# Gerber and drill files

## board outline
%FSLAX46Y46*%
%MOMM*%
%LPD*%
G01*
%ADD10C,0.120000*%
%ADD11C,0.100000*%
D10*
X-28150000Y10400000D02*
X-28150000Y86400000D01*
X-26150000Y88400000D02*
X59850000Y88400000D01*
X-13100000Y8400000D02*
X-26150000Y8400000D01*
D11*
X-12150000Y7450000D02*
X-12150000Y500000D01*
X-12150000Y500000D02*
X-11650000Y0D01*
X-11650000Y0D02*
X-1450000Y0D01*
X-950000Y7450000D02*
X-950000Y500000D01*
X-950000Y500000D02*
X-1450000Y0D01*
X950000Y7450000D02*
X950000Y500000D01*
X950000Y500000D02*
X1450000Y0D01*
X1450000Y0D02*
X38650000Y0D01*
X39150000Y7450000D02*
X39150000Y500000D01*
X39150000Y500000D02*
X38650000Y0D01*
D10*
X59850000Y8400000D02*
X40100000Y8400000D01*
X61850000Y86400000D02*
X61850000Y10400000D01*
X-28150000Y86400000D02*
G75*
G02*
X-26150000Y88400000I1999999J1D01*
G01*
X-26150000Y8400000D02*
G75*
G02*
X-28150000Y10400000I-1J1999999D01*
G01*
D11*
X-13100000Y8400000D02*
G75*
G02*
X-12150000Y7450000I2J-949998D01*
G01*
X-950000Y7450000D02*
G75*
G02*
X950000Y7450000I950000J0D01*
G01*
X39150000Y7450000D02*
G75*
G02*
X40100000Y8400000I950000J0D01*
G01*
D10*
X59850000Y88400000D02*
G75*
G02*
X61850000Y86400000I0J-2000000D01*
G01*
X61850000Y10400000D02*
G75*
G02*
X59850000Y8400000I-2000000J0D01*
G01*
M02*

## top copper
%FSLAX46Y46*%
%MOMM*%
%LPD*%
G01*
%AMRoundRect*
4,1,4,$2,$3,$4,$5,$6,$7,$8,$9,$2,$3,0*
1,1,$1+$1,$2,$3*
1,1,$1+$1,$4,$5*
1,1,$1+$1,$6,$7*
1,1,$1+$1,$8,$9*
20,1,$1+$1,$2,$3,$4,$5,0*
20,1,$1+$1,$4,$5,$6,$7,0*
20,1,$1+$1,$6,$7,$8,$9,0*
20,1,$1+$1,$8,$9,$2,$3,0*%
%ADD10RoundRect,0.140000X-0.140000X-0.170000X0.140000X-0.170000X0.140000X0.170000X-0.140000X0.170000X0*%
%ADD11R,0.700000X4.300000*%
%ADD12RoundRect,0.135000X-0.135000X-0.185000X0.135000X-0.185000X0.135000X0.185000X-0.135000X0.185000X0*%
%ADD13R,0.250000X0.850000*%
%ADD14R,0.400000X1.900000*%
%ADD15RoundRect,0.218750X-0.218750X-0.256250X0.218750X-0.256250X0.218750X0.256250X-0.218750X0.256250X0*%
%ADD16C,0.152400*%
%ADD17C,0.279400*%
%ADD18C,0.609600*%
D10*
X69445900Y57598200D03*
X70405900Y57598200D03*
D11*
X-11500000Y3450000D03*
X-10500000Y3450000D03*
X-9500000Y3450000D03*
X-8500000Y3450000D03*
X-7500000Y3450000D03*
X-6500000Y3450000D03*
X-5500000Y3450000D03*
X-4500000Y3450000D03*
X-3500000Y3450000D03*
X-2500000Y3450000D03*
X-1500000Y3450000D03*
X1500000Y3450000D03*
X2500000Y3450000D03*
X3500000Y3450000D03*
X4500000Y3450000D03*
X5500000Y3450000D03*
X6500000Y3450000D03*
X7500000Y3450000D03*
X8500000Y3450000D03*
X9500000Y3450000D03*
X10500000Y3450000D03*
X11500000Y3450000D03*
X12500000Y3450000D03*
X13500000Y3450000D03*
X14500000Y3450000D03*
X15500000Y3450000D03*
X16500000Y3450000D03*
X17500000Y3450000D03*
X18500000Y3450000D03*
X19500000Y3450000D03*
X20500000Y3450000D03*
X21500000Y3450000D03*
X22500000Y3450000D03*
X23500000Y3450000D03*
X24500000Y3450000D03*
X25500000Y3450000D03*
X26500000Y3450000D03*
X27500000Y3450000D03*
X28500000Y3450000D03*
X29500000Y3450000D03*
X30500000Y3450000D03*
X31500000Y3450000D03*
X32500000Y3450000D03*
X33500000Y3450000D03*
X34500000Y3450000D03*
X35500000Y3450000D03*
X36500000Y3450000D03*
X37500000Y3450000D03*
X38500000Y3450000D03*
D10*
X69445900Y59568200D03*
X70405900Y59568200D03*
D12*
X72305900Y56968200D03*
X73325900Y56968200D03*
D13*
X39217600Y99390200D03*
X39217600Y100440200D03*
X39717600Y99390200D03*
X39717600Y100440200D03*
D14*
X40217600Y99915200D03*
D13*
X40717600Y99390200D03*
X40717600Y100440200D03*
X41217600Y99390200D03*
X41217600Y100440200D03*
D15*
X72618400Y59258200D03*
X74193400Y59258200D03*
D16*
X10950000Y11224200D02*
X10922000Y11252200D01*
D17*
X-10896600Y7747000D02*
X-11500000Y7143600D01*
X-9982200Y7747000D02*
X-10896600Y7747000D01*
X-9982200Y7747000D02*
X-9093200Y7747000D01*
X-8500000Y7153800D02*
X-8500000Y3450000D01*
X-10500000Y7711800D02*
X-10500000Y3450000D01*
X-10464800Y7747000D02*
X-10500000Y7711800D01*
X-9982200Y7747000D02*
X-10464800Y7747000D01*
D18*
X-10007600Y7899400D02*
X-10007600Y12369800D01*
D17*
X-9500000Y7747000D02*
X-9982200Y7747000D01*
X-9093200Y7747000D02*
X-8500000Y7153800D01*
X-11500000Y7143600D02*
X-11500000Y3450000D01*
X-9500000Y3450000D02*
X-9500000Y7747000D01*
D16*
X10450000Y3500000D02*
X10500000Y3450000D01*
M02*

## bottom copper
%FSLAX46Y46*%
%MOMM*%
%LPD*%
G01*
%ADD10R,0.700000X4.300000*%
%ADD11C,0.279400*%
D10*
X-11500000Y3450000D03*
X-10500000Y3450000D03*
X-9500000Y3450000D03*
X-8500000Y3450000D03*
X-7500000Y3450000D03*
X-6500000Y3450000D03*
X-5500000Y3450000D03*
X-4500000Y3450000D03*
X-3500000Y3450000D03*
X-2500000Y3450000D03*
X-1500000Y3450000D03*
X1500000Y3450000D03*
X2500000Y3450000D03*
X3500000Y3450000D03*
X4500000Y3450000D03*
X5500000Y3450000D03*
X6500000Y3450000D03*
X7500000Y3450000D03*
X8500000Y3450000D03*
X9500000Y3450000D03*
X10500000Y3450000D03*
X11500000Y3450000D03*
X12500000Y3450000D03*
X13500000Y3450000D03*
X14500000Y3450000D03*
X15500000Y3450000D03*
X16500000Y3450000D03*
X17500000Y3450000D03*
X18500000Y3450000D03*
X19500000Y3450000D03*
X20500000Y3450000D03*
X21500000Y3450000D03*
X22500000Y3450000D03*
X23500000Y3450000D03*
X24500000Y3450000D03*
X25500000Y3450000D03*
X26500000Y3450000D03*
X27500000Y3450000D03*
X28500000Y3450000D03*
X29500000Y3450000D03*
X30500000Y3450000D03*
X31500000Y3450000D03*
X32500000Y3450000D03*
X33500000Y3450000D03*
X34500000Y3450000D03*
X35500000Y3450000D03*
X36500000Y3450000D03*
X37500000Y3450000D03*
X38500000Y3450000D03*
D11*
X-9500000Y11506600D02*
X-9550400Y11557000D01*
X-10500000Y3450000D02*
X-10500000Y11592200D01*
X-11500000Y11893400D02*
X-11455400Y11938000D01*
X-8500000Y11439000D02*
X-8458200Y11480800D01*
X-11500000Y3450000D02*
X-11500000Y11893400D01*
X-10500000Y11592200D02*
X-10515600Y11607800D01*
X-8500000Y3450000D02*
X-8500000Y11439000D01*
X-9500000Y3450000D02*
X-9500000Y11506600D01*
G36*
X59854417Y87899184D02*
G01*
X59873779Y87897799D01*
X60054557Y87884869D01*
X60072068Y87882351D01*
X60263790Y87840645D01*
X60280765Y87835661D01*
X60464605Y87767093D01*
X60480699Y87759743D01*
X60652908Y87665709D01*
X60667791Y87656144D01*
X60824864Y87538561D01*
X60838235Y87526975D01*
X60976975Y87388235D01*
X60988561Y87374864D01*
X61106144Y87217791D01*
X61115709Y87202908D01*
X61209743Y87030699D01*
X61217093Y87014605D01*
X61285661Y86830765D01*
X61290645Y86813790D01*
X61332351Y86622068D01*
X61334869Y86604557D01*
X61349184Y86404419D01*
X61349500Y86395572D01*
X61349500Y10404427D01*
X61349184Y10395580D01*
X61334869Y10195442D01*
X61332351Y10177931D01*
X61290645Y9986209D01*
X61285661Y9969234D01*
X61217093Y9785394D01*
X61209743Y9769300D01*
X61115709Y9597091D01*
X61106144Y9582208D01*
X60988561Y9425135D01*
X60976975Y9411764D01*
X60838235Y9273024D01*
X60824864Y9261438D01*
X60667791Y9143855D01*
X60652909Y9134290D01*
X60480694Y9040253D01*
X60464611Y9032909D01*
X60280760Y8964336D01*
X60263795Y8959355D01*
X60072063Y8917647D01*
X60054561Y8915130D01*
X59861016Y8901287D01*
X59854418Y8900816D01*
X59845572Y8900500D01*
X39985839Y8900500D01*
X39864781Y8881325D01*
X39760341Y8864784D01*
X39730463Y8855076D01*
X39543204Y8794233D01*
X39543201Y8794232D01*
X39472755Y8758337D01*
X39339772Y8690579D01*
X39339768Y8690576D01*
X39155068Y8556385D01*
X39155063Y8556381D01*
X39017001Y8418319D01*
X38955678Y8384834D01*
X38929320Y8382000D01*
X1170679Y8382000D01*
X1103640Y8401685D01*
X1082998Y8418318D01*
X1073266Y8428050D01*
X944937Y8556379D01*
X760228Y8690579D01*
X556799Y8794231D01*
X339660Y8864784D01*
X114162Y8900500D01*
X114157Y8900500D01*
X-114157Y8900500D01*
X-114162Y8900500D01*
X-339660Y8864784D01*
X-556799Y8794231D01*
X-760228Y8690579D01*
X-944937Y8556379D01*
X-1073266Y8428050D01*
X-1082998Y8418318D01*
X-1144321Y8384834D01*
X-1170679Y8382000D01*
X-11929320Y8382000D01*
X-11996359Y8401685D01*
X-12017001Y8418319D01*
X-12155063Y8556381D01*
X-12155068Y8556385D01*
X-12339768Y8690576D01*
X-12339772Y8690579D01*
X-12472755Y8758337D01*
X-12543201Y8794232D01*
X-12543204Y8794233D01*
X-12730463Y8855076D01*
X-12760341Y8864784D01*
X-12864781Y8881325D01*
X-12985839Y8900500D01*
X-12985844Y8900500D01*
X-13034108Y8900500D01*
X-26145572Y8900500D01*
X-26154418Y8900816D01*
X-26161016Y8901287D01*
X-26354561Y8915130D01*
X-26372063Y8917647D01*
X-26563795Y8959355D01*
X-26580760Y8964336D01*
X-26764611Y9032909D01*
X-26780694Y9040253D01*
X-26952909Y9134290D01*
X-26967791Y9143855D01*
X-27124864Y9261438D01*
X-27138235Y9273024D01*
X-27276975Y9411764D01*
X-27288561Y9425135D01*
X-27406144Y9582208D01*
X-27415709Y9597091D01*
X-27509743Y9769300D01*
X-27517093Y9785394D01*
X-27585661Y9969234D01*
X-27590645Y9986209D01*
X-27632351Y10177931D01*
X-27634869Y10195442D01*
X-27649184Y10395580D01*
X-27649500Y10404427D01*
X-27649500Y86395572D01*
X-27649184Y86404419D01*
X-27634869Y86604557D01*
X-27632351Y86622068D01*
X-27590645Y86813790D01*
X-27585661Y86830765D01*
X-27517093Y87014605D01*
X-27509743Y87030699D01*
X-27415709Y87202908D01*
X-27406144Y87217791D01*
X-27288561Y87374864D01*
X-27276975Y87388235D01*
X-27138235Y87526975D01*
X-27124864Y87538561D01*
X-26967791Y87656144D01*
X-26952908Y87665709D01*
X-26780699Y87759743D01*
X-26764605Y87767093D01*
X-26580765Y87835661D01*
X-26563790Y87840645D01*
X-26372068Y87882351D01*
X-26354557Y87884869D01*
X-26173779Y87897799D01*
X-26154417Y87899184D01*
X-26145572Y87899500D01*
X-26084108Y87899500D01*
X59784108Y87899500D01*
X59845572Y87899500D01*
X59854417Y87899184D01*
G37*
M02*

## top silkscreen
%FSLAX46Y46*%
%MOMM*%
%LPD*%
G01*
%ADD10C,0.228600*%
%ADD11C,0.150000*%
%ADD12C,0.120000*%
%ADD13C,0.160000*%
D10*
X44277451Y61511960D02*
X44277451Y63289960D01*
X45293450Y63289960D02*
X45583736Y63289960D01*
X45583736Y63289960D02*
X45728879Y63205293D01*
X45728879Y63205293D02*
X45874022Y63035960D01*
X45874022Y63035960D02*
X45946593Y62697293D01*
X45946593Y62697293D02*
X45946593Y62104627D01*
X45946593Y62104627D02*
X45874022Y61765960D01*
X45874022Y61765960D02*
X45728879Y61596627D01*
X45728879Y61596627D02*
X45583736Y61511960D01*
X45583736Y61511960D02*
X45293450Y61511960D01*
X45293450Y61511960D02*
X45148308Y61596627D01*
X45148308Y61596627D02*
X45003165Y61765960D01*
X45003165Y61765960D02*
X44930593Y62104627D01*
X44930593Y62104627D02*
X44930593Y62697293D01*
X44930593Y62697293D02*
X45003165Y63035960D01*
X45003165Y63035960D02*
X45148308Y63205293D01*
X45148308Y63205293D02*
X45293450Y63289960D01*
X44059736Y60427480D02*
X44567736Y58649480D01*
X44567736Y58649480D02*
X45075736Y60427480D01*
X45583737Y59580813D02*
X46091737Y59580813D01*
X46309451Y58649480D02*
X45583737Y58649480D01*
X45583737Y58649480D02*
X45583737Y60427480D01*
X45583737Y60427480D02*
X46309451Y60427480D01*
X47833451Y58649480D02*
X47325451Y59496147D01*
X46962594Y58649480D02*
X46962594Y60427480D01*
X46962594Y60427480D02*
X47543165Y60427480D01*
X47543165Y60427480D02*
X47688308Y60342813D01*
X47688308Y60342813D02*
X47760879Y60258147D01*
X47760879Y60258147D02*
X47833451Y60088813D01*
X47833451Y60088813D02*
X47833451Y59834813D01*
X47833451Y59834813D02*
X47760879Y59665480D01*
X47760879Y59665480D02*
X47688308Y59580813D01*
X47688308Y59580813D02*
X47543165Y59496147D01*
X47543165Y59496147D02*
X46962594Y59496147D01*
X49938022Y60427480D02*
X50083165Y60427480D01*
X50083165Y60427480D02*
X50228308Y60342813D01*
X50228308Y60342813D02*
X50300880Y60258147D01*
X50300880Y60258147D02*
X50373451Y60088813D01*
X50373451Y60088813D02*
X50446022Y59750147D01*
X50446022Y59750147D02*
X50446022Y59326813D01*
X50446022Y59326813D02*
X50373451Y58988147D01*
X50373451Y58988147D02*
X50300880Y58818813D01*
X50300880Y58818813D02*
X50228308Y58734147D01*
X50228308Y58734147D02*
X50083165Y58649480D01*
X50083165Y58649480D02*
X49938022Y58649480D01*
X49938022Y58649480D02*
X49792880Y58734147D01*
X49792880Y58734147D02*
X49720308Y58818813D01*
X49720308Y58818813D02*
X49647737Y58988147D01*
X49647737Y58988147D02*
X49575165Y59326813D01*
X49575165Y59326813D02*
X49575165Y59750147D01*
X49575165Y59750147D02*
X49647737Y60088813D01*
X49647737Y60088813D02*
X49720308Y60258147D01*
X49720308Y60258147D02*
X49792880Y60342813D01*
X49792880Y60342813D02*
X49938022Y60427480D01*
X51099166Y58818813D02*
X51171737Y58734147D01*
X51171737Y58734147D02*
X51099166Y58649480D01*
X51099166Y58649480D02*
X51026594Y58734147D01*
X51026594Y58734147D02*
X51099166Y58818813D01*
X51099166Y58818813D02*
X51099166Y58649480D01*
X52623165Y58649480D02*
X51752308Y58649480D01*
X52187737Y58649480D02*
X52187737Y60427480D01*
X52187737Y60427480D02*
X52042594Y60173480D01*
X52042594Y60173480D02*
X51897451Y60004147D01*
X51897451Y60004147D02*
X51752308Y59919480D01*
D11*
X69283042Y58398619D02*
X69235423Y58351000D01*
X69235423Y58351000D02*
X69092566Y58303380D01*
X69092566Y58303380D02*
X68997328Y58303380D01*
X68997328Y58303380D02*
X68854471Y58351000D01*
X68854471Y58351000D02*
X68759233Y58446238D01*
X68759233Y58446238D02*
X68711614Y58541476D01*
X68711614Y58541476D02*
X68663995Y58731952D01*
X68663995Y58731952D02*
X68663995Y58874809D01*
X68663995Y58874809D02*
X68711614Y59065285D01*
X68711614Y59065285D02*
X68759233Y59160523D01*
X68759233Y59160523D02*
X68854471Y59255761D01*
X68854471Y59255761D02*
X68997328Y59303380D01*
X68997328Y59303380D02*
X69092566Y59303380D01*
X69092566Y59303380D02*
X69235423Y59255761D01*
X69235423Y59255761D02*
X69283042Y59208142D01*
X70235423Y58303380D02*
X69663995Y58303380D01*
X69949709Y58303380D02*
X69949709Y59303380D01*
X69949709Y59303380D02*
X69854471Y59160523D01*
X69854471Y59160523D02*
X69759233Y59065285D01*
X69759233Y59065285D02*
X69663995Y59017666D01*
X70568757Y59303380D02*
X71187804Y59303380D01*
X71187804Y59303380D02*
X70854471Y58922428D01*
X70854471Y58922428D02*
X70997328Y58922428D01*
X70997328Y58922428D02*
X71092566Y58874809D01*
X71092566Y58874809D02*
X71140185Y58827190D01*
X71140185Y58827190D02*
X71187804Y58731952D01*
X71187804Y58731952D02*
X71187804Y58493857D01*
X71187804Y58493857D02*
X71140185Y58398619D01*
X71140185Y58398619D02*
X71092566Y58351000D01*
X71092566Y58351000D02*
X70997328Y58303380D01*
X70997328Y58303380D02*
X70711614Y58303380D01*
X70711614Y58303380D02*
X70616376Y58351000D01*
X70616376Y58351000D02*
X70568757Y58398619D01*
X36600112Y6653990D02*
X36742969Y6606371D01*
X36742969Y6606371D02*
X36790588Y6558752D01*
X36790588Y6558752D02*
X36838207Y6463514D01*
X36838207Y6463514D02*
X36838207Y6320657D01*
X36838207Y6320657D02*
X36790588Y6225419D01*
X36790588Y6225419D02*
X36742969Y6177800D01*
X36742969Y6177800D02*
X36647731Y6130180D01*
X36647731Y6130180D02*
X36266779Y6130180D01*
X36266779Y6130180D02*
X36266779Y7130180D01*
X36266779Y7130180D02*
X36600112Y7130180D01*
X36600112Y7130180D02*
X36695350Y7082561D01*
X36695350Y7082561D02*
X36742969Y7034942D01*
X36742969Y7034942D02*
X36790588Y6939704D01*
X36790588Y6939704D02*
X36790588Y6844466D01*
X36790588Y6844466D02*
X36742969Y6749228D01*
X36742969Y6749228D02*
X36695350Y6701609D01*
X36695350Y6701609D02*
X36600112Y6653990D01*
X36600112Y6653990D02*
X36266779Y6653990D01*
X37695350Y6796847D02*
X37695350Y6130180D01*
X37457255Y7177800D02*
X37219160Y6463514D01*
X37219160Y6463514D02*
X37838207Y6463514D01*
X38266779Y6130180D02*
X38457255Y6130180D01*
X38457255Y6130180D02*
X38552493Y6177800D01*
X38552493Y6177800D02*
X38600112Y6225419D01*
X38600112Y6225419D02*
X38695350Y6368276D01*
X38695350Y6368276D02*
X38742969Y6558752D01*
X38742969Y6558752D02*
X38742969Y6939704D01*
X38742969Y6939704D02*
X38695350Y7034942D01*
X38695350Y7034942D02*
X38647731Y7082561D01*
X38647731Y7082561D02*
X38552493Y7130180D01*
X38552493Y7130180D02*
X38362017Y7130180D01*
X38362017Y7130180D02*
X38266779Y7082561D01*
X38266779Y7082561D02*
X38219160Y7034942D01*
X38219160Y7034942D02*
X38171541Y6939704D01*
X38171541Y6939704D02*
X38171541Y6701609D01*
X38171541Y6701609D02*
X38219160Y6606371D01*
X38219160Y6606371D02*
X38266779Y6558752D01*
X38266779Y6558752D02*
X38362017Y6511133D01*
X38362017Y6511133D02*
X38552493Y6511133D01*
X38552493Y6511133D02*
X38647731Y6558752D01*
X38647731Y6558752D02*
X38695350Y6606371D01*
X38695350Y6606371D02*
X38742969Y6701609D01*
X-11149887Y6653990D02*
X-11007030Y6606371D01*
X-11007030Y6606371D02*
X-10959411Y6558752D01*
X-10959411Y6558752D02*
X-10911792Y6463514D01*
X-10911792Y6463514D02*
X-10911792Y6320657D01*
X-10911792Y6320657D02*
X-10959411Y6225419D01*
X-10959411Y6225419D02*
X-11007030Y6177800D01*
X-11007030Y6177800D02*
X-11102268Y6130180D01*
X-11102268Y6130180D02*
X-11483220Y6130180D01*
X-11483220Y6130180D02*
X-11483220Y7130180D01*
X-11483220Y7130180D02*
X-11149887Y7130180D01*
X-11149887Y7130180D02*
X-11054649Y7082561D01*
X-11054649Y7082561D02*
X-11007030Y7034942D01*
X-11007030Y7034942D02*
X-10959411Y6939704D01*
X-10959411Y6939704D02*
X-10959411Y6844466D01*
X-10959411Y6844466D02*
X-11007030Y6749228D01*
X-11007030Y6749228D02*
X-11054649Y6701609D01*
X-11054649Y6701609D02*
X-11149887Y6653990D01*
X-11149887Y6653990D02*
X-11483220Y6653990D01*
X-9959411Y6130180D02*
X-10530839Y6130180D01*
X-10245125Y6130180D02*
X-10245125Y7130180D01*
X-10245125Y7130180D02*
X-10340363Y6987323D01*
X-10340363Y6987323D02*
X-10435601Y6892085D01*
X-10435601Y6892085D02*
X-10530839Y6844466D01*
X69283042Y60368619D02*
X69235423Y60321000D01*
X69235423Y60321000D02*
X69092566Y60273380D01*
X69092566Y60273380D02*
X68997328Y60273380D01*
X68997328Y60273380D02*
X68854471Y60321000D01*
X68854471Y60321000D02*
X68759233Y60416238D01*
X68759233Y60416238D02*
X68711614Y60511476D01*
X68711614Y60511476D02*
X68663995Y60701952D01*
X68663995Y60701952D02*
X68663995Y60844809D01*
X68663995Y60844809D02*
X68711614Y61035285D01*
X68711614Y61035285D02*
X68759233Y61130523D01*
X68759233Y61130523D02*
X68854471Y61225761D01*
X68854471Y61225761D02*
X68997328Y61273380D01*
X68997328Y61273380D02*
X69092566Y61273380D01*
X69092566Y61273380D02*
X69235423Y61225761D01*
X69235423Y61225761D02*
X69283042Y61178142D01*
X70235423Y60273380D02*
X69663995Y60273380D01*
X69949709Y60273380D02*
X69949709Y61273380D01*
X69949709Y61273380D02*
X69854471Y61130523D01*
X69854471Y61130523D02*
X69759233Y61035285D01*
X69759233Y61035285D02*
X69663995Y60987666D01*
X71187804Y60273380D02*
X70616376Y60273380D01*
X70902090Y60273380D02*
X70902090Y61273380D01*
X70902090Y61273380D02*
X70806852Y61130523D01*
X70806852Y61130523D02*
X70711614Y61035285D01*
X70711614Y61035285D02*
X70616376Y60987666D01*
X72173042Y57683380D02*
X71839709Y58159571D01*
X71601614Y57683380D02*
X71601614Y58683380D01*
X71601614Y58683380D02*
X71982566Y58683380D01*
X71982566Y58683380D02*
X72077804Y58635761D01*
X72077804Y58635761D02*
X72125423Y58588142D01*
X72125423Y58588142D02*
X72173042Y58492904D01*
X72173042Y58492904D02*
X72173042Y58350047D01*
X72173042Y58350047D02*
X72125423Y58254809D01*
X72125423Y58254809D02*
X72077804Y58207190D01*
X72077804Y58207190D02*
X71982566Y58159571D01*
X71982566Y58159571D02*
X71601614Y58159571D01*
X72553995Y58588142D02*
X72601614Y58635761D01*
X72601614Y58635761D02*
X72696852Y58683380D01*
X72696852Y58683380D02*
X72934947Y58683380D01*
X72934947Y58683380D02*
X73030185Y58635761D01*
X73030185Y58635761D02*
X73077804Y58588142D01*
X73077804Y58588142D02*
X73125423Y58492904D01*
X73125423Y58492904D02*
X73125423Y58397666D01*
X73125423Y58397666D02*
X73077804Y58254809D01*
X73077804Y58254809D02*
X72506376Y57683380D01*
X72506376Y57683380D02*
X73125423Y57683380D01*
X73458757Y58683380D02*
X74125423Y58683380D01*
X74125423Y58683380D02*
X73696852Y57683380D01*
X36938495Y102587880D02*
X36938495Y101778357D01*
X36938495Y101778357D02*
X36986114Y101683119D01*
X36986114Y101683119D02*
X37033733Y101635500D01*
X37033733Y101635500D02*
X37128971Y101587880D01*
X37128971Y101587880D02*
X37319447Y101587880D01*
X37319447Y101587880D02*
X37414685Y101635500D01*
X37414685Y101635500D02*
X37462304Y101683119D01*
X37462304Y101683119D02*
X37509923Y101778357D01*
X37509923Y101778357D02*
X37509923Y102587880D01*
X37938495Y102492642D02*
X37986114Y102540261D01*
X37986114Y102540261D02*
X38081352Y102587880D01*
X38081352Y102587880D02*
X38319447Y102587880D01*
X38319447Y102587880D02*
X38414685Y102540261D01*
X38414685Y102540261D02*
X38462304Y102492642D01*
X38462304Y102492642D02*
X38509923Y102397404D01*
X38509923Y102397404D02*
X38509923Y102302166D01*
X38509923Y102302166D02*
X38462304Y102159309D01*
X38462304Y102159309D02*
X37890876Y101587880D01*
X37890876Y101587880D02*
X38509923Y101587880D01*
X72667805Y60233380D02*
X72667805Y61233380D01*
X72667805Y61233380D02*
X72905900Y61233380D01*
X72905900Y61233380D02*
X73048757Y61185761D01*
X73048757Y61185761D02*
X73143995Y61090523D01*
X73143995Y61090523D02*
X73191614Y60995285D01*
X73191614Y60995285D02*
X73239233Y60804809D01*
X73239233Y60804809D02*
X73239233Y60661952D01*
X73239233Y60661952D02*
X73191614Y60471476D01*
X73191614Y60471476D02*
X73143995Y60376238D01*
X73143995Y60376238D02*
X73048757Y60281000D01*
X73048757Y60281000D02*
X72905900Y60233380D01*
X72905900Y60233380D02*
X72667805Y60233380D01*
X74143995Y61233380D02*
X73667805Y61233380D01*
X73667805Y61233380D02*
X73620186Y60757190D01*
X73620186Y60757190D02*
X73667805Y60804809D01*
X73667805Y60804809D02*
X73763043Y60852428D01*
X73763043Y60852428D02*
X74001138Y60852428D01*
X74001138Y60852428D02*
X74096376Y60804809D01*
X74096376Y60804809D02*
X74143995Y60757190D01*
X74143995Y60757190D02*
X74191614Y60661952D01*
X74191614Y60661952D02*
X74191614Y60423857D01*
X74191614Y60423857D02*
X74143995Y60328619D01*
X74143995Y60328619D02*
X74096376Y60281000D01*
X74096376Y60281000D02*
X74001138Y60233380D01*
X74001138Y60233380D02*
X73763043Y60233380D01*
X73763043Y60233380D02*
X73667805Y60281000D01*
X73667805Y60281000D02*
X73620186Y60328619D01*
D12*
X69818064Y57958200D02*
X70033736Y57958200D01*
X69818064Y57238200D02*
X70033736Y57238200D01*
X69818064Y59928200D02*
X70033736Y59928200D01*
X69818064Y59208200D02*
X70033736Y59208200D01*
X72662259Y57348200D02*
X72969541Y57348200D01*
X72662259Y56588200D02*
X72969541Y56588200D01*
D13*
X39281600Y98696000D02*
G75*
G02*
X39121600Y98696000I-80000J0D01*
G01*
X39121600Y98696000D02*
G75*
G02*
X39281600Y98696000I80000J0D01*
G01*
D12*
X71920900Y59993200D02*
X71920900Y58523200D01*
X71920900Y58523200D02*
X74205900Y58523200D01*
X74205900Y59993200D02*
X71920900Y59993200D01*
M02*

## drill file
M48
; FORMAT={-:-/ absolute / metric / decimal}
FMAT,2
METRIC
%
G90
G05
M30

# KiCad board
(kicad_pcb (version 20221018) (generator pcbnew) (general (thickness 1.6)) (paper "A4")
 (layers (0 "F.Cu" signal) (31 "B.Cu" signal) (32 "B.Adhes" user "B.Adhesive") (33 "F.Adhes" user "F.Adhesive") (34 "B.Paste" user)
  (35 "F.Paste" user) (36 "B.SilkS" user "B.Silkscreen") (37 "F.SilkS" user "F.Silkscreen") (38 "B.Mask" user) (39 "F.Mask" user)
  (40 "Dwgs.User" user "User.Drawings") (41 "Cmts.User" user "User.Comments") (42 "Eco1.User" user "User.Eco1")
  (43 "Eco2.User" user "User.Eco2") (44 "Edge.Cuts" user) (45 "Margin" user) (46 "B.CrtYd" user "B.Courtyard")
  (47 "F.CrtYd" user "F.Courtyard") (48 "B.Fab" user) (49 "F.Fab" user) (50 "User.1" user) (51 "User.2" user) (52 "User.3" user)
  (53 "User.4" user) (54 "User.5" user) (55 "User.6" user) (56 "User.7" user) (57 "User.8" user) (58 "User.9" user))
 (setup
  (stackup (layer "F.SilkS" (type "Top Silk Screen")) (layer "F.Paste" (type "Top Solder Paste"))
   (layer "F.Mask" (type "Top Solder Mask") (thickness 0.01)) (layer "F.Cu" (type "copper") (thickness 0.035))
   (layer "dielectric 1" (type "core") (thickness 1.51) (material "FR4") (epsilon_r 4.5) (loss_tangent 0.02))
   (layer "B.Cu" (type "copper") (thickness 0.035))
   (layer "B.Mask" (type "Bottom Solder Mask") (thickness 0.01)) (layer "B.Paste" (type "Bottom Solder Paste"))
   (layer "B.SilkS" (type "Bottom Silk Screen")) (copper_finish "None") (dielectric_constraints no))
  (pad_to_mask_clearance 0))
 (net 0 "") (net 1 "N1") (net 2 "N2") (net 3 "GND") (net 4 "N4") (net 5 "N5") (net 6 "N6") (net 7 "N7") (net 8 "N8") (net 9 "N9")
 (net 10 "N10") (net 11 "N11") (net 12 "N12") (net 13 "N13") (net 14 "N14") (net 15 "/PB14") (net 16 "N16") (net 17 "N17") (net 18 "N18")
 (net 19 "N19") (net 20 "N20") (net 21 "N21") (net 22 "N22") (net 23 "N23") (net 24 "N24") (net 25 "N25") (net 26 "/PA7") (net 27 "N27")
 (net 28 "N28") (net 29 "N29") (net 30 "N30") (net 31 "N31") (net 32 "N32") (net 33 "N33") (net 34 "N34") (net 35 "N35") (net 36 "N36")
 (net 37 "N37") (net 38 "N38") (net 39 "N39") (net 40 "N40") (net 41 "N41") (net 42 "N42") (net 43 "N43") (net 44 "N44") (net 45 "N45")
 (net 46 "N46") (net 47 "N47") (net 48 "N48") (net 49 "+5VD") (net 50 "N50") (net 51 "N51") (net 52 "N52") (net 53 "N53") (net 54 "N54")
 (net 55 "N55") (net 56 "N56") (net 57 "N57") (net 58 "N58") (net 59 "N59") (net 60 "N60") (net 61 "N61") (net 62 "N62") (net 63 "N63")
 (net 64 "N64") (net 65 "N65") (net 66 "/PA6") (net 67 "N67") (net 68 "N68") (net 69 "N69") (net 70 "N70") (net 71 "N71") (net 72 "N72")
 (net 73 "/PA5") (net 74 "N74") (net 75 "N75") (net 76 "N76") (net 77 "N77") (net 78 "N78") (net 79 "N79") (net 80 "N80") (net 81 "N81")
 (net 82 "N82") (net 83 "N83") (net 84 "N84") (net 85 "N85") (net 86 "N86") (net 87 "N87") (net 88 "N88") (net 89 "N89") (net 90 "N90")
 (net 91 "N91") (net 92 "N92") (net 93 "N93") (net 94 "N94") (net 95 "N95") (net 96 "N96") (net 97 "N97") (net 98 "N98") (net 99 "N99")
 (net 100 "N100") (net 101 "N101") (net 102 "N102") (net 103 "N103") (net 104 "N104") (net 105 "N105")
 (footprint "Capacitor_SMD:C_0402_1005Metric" (layer "F.Cu") (at 69.9259 -57.5982)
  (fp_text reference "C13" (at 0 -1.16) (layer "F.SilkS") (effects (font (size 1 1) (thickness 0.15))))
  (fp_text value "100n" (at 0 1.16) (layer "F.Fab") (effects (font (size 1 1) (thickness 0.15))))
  (fp_line (start -0.107836 -0.36) (end 0.107836 -0.36) (stroke (width 0.12) (type solid)) (layer "F.SilkS"))
  (fp_line (start -0.107836 0.36) (end 0.107836 0.36) (stroke (width 0.12) (type solid)) (layer "F.SilkS"))
  (pad "1" smd roundrect (at -0.48 0) (size 0.56 0.62) (layers "F.Cu" "F.Paste" "F.Mask") (roundrect_rratio 0.25) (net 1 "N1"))
  (pad "2" smd roundrect (at 0.48 0) (size 0.56 0.62) (layers "F.Cu" "F.Paste" "F.Mask") (roundrect_rratio 0.25) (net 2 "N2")))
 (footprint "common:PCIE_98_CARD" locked (layer "F.Cu") (at 0 0)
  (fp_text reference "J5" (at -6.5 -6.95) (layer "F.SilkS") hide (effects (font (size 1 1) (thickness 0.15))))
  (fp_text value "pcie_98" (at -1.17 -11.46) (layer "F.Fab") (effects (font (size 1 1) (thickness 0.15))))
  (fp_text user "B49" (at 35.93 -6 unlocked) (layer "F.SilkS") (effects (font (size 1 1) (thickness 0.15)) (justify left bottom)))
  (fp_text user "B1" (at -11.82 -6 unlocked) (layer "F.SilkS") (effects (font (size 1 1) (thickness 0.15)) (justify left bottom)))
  (fp_line (start -28.15 -10.4) (end -28.15 -86.4) (stroke (width 0.12) (type default)) (layer "Edge.Cuts"))
  (fp_line (start -26.15 -88.4) (end 59.85 -88.4) (stroke (width 0.12) (type default)) (layer "Edge.Cuts"))
  (fp_line (start -13.1 -8.4) (end -26.15 -8.4) (stroke (width 0.12) (type default)) (layer "Edge.Cuts"))
  (fp_line (start -12.15 -7.45) (end -12.15 -0.5) (stroke (width 0.1) (type solid)) (layer "Edge.Cuts"))
  (fp_line (start -12.15 -0.5) (end -11.65 0) (stroke (width 0.1) (type solid)) (layer "Edge.Cuts"))
  (fp_line (start -11.65 0) (end -1.45 0) (stroke (width 0.1) (type solid)) (layer "Edge.Cuts"))
  (fp_line (start -0.95 -7.45) (end -0.95 -0.5) (stroke (width 0.1) (type solid)) (layer "Edge.Cuts"))
  (fp_line (start -0.95 -0.5) (end -1.45 0) (stroke (width 0.1) (type solid)) (layer "Edge.Cuts"))
  (fp_line (start 0.95 -7.45) (end 0.95 -0.5) (stroke (width 0.1) (type solid)) (layer "Edge.Cuts"))
  (fp_line (start 0.95 -0.5) (end 1.45 0) (stroke (width 0.1) (type solid)) (layer "Edge.Cuts"))
  (fp_line (start 1.45 0) (end 38.65 0) (stroke (width 0.1) (type solid)) (layer "Edge.Cuts"))
  (fp_line (start 39.15 -7.45) (end 39.15 -0.5) (stroke (width 0.1) (type solid)) (layer "Edge.Cuts"))
  (fp_line (start 39.15 -0.5) (end 38.65 0) (stroke (width 0.1) (type solid)) (layer "Edge.Cuts"))
  (fp_line (start 59.85 -8.4) (end 40.1 -8.4) (stroke (width 0.12) (type default)) (layer "Edge.Cuts"))
  (fp_line (start 61.85 -86.4) (end 61.85 -10.4) (stroke (width 0.12) (type default)) (layer "Edge.Cuts"))
  (fp_arc (start -28.15 -86.4) (mid -27.564214 -87.814214) (end -26.15 -88.4) (stroke (width 0.12) (type default)) (layer "Edge.Cuts"))
  (fp_arc (start -26.15 -8.4) (mid -27.564214 -8.985786) (end -28.15 -10.4) (stroke (width 0.12) (type default)) (layer "Edge.Cuts"))
  (fp_arc (start -13.1 -8.4) (mid -12.428248 -8.121752) (end -12.15 -7.45) (stroke (width 0.1) (type default)) (layer "Edge.Cuts"))
  (fp_arc (start -0.95 -7.45) (mid 0 -8.4) (end 0.95 -7.45) (stroke (width 0.1) (type solid)) (layer "Edge.Cuts"))
  (fp_arc (start 39.15 -7.45) (mid 39.428248 -8.121752) (end 40.1 -8.4) (stroke (width 0.1) (type default)) (layer "Edge.Cuts"))
  (fp_arc (start 59.85 -88.4) (mid 61.264214 -87.814214) (end 61.85 -86.4) (stroke (width 0.12) (type default)) (layer "Edge.Cuts"))
  (fp_arc (start 61.85 -10.4) (mid 61.264214 -8.985786) (end 59.85 -8.4) (stroke (width 0.12) (type default)) (layer "Edge.Cuts"))
  (pad "A1" connect rect locked (at -11.5 -3.45) (size 0.7 4.3) (layers "B.Cu" "B.Mask") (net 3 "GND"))
  (pad "A2" connect rect locked (at -10.5 -3.45) (size 0.7 4.3) (layers "B.Cu" "B.Mask") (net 3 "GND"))
  (pad "A3" connect rect locked (at -9.5 -3.45) (size 0.7 4.3) (layers "B.Cu" "B.Mask") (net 3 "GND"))
  (pad "A4" connect rect locked (at -8.5 -3.45) (size 0.7 4.3) (layers "B.Cu" "B.Mask") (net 3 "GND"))
  (pad "A5" connect rect locked (at -7.5 -3.45) (size 0.7 4.3) (layers "B.Cu" "B.Mask") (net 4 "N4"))
  (pad "A6" connect rect locked (at -6.5 -3.45) (size 0.7 4.3) (layers "B.Cu" "B.Mask") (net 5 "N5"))
  (pad "A7" connect rect locked (at -5.5 -3.45) (size 0.7 4.3) (layers "B.Cu" "B.Mask") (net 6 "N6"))
  (pad "A8" connect rect locked (at -4.5 -3.45) (size 0.7 4.3) (layers "B.Cu" "B.Mask") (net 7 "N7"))
  (pad "A9" connect rect locked (at -3.5 -3.45) (size 0.7 4.3) (layers "B.Cu" "B.Mask") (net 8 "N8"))
  (pad "A10" connect rect locked (at -2.5 -3.45) (size 0.7 4.3) (layers "B.Cu" "B.Mask") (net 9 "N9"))
  (pad "A11" connect rect locked (at -1.5 -3.45) (size 0.7 4.3) (layers "B.Cu" "B.Mask") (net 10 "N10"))
  (pad "A12" connect rect locked (at 1.5 -3.45) (size 0.7 4.3) (layers "B.Cu" "B.Mask") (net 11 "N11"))
  (pad "A13" connect rect locked (at 2.5 -3.45) (size 0.7 4.3) (layers "B.Cu" "B.Mask") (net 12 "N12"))
  (pad "A14" connect rect locked (at 3.5 -3.45) (size 0.7 4.3) (layers "B.Cu" "B.Mask") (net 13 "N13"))
  (pad "A15" connect rect locked (at 4.5 -3.45) (size 0.7 4.3) (layers "B.Cu" "B.Mask") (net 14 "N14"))
  (pad "A16" connect rect locked (at 5.5 -3.45) (size 0.7 4.3) (layers "B.Cu" "B.Mask") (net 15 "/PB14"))
  (pad "A17" connect rect locked (at 6.5 -3.45) (size 0.7 4.3) (layers "B.Cu" "B.Mask") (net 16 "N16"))
  (pad "A18" connect rect locked (at 7.5 -3.45) (size 0.7 4.3) (layers "B.Cu" "B.Mask") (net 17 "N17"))
  (pad "A19" connect rect locked (at 8.5 -3.45) (size 0.7 4.3) (layers "B.Cu" "B.Mask") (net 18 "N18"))
  (pad "A20" connect rect locked (at 9.5 -3.45) (size 0.7 4.3) (layers "B.Cu" "B.Mask") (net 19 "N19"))
  (pad "A21" connect rect locked (at 10.5 -3.45) (size 0.7 4.3) (layers "B.Cu" "B.Mask") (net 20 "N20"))
  (pad "A22" connect rect locked (at 11.5 -3.45) (size 0.7 4.3) (layers "B.Cu" "B.Mask") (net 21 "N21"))
  (pad "A23" connect rect locked (at 12.5 -3.45) (size 0.7 4.3) (layers "B.Cu" "B.Mask") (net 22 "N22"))
  (pad "A24" connect rect locked (at 13.5 -3.45) (size 0.7 4.3) (layers "B.Cu" "B.Mask") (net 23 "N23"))
  (pad "A25" connect rect locked (at 14.5 -3.45) (size 0.7 4.3) (layers "B.Cu" "B.Mask") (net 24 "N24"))
  (pad "A26" connect rect locked (at 15.5 -3.45) (size 0.7 4.3) (layers "B.Cu" "B.Mask") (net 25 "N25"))
  (pad "A27" connect rect locked (at 16.5 -3.45) (size 0.7 4.3) (layers "B.Cu" "B.Mask") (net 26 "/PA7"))
  (pad "A28" connect rect locked (at 17.5 -3.45) (size 0.7 4.3) (layers "B.Cu" "B.Mask") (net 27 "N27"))
  (pad "A29" connect rect locked (at 18.5 -3.45) (size 0.7 4.3) (layers "B.Cu" "B.Mask") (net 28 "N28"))
  (pad "A30" connect rect locked (at 19.5 -3.45) (size 0.7 4.3) (layers "B.Cu" "B.Mask") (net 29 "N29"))
  (pad "A31" connect rect locked (at 20.5 -3.45) (size 0.7 4.3) (layers "B.Cu" "B.Mask") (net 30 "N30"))
  (pad "A32" connect rect locked (at 21.5 -3.45) (size 0.7 4.3) (layers "B.Cu" "B.Mask") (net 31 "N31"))
  (pad "A33" connect rect locked (at 22.5 -3.45) (size 0.7 4.3) (layers "B.Cu" "B.Mask") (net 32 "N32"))
  (pad "A34" connect rect locked (at 23.5 -3.45) (size 0.7 4.3) (layers "B.Cu" "B.Mask") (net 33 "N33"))
  (pad "A35" connect rect locked (at 24.5 -3.45) (size 0.7 4.3) (layers "B.Cu" "B.Mask") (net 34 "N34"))
  (pad "A36" connect rect locked (at 25.5 -3.45) (size 0.7 4.3) (layers "B.Cu" "B.Mask") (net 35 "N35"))
  (pad "A37" connect rect locked (at 26.5 -3.45) (size 0.7 4.3) (layers "B.Cu" "B.Mask") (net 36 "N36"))
  (pad "A38" connect rect locked (at 27.5 -3.45) (size 0.7 4.3) (layers "B.Cu" "B.Mask") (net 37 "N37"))
  (pad "A39" connect rect locked (at 28.5 -3.45) (size 0.7 4.3) (layers "B.Cu" "B.Mask") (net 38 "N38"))
  (pad "A40" connect rect locked (at 29.5 -3.45) (size 0.7 4.3) (layers "B.Cu" "B.Mask") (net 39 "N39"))
  (pad "A41" connect rect locked (at 30.5 -3.45) (size 0.7 4.3) (layers "B.Cu" "B.Mask") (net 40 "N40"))
  (pad "A42" connect rect locked (at 31.5 -3.45) (size 0.7 4.3) (layers "B.Cu" "B.Mask") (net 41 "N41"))
  (pad "A43" connect rect locked (at 32.5 -3.45) (size 0.7 4.3) (layers "B.Cu" "B.Mask") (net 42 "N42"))
  (pad "A44" connect rect locked (at 33.5 -3.45) (size 0.7 4.3) (layers "B.Cu" "B.Mask") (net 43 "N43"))
  (pad "A45" connect rect locked (at 34.5 -3.45) (size 0.7 4.3) (layers "B.Cu" "B.Mask") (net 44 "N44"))
  (pad "A46" connect rect locked (at 35.5 -3.45) (size 0.7 4.3) (layers "B.Cu" "B.Mask") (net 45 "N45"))
  (pad "A47" connect rect locked (at 36.5 -3.45) (size 0.7 4.3) (layers "B.Cu" "B.Mask") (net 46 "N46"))
  (pad "A48" connect rect locked (at 37.5 -3.45) (size 0.7 4.3) (layers "B.Cu" "B.Mask") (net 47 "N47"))
  (pad "A49" connect rect locked (at 38.5 -3.45) (size 0.7 4.3) (layers "B.Cu" "B.Mask") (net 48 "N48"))
  (pad "B1" connect rect locked (at -11.5 -3.45) (size 0.7 4.3) (layers "F.Cu" "F.Mask") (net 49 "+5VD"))
  (pad "B2" connect rect locked (at -10.5 -3.45) (size 0.7 4.3) (layers "F.Cu" "F.Mask") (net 49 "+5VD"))
  (pad "B3" connect rect locked (at -9.5 -3.45) (size 0.7 4.3) (layers "F.Cu" "F.Mask") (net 49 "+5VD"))
  (pad "B4" connect rect locked (at -8.5 -3.45) (size 0.7 4.3) (layers "F.Cu" "F.Mask") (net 49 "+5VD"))
  (pad "B5" connect rect locked (at -7.5 -3.45) (size 0.7 4.3) (layers "F.Cu" "F.Mask") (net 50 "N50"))
  (pad "B6" connect rect locked (at -6.5 -3.45) (size 0.7 4.3) (layers "F.Cu" "F.Mask") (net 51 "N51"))
  (pad "B7" connect rect locked (at -5.5 -3.45) (size 0.7 4.3) (layers "F.Cu" "F.Mask") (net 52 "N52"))
  (pad "B8" connect rect locked (at -4.5 -3.45) (size 0.7 4.3) (layers "F.Cu" "F.Mask") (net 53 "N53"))
  (pad "B9" connect rect locked (at -3.5 -3.45) (size 0.7 4.3) (layers "F.Cu" "F.Mask") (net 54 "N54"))
  (pad "B10" connect rect locked (at -2.5 -3.45) (size 0.7 4.3) (layers "F.Cu" "F.Mask") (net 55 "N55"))
  (pad "B11" connect rect locked (at -1.5 -3.45) (size 0.7 4.3) (layers "F.Cu" "F.Mask") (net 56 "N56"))
  (pad "B12" connect rect locked (at 1.5 -3.45) (size 0.7 4.3) (layers "F.Cu" "F.Mask") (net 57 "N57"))
  (pad "B13" connect rect locked (at 2.5 -3.45) (size 0.7 4.3) (layers "F.Cu" "F.Mask") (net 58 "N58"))
  (pad "B14" connect rect locked (at 3.5 -3.45) (size 0.7 4.3) (layers "F.Cu" "F.Mask") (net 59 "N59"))
  (pad "B15" connect rect locked (at 4.5 -3.45) (size 0.7 4.3) (layers "F.Cu" "F.Mask") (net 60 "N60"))
  (pad "B16" connect rect locked (at 5.5 -3.45) (size 0.7 4.3) (layers "F.Cu" "F.Mask") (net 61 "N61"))
  (pad "B17" connect rect locked (at 6.5 -3.45) (size 0.7 4.3) (layers "F.Cu" "F.Mask") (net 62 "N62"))
  (pad "B18" connect rect locked (at 7.5 -3.45) (size 0.7 4.3) (layers "F.Cu" "F.Mask") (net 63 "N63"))
  (pad "B19" connect rect locked (at 8.5 -3.45) (size 0.7 4.3) (layers "F.Cu" "F.Mask") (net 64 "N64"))
  (pad "B20" connect rect locked (at 9.5 -3.45) (size 0.7 4.3) (layers "F.Cu" "F.Mask") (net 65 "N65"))
  (pad "B21" connect rect locked (at 10.5 -3.45) (size 0.7 4.3) (layers "F.Cu" "F.Mask") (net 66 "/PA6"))
  (pad "B22" connect rect locked (at 11.5 -3.45) (size 0.7 4.3) (layers "F.Cu" "F.Mask") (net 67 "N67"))
  (pad "B23" connect rect locked (at 12.5 -3.45) (size 0.7 4.3) (layers "F.Cu" "F.Mask") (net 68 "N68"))
  (pad "B24" connect rect locked (at 13.5 -3.45) (size 0.7 4.3) (layers "F.Cu" "F.Mask") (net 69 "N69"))
  (pad "B25" connect rect locked (at 14.5 -3.45) (size 0.7 4.3) (layers "F.Cu" "F.Mask") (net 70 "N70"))
  (pad "B26" connect rect locked (at 15.5 -3.45) (size 0.7 4.3) (layers "F.Cu" "F.Mask") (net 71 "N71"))
  (pad "B27" connect rect locked (at 16.5 -3.45) (size 0.7 4.3) (layers "F.Cu" "F.Mask") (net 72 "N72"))
  (pad "B28" connect rect locked (at 17.5 -3.45) (size 0.7 4.3) (layers "F.Cu" "F.Mask") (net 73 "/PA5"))
  (pad "B29" connect rect locked (at 18.5 -3.45) (size 0.7 4.3) (layers "F.Cu" "F.Mask") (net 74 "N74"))
  (pad "B30" connect rect locked (at 19.5 -3.45) (size 0.7 4.3) (layers "F.Cu" "F.Mask") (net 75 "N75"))
  (pad "B31" connect rect locked (at 20.5 -3.45) (size 0.7 4.3) (layers "F.Cu" "F.Mask") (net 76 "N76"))
  (pad "B32" connect rect locked (at 21.5 -3.45) (size 0.7 4.3) (layers "F.Cu" "F.Mask") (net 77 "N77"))
  (pad "B33" connect rect locked (at 22.5 -3.45) (size 0.7 4.3) (layers "F.Cu" "F.Mask") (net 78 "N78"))
  (pad "B34" connect rect locked (at 23.5 -3.45) (size 0.7 4.3) (layers "F.Cu" "F.Mask") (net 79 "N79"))
  (pad "B35" connect rect locked (at 24.5 -3.45) (size 0.7 4.3) (layers "F.Cu" "F.Mask") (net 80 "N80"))
  (pad "B36" connect rect locked (at 25.5 -3.45) (size 0.7 4.3) (layers "F.Cu" "F.Mask") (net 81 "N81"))
  (pad "B37" connect rect locked (at 26.5 -3.45) (size 0.7 4.3) (layers "F.Cu" "F.Mask") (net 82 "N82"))
  (pad "B38" connect rect locked (at 27.5 -3.45) (size 0.7 4.3) (layers "F.Cu" "F.Mask") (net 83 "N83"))
  (pad "B39" connect rect locked (at 28.5 -3.45) (size 0.7 4.3) (layers "F.Cu" "F.Mask") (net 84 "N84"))
  (pad "B40" connect rect locked (at 29.5 -3.45) (size 0.7 4.3) (layers "F.Cu" "F.Mask") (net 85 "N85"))
  (pad "B41" connect rect locked (at 30.5 -3.45) (size 0.7 4.3) (layers "F.Cu" "F.Mask") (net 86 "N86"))
  (pad "B42" connect rect locked (at 31.5 -3.45) (size 0.7 4.3) (layers "F.Cu" "F.Mask") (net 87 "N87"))
  (pad "B43" connect rect locked (at 32.5 -3.45) (size 0.7 4.3) (layers "F.Cu" "F.Mask") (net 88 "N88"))
  (pad "B44" connect rect locked (at 33.5 -3.45) (size 0.7 4.3) (layers "F.Cu" "F.Mask") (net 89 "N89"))
  (pad "B45" connect rect locked (at 34.5 -3.45) (size 0.7 4.3) (layers "F.Cu" "F.Mask") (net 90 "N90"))
  (pad "B46" connect rect locked (at 35.5 -3.45) (size 0.7 4.3) (layers "F.Cu" "F.Mask") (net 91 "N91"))
  (pad "B47" connect rect locked (at 36.5 -3.45) (size 0.7 4.3) (layers "F.Cu" "F.Mask") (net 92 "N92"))
  (pad "B48" connect rect locked (at 37.5 -3.45) (size 0.7 4.3) (layers "F.Cu" "F.Mask") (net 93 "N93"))
  (pad "B49" connect rect locked (at 38.5 -3.45) (size 0.7 4.3) (layers "F.Cu" "F.Mask") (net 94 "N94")))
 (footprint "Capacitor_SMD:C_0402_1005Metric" (layer "F.Cu") (at 69.9259 -59.5682)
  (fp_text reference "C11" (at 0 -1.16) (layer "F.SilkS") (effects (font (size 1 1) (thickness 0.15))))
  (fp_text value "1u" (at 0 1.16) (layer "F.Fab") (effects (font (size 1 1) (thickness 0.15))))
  (fp_line (start -0.107836 -0.36) (end 0.107836 -0.36) (stroke (width 0.12) (type solid)) (layer "F.SilkS"))
  (fp_line (start -0.107836 0.36) (end 0.107836 0.36) (stroke (width 0.12) (type solid)) (layer "F.SilkS"))
  (pad "1" smd roundrect (at -0.48 0) (size 0.56 0.62) (layers "F.Cu" "F.Paste" "F.Mask") (roundrect_rratio 0.25) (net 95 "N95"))
  (pad "2" smd roundrect (at 0.48 0) (size 0.56 0.62) (layers "F.Cu" "F.Paste" "F.Mask") (roundrect_rratio 0.25) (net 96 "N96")))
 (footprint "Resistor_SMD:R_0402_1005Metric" (layer "F.Cu") (at 72.8159 -56.9682)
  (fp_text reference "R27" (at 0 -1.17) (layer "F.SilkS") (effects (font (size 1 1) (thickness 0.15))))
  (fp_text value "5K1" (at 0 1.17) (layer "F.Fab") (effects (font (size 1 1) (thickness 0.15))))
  (fp_line (start -0.153641 -0.38) (end 0.153641 -0.38) (stroke (width 0.12) (type solid)) (layer "F.SilkS"))
  (fp_line (start -0.153641 0.38) (end 0.153641 0.38) (stroke (width 0.12) (type solid)) (layer "F.SilkS"))
  (pad "1" smd roundrect (at -0.51 0) (size 0.54 0.64) (layers "F.Cu" "F.Paste" "F.Mask") (roundrect_rratio 0.25) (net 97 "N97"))
  (pad "2" smd roundrect (at 0.51 0) (size 0.54 0.64) (layers "F.Cu" "F.Paste" "F.Mask") (roundrect_rratio 0.25) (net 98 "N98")))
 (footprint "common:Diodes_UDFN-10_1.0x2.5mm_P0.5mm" (layer "F.Cu") (at 40.2176 -99.9152 90)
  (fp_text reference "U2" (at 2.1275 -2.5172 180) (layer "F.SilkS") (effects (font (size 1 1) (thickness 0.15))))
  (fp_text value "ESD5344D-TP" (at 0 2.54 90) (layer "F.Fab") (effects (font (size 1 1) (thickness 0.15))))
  (fp_circle (center -1.2192 -1.016) (end -1.1192 -1.016) (stroke (width 0.12) (type solid)) (fill solid) (layer "F.SilkS"))
  (pad "1" smd rect (at -0.525 -1) (size 0.25 0.85) (layers "F.Cu" "F.Paste" "F.Mask") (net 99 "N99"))
  (pad "1" smd rect (at 0.525 -1) (size 0.25 0.85) (layers "F.Cu" "F.Paste" "F.Mask") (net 99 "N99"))
  (pad "2" smd rect (at -0.525 -0.5) (size 0.25 0.85) (layers "F.Cu" "F.Paste" "F.Mask") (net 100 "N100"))
  (pad "2" smd rect (at 0.525 -0.5) (size 0.25 0.85) (layers "F.Cu" "F.Paste" "F.Mask") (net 100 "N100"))
  (pad "3" smd rect (at 0 0) (size 0.4 1.9) (layers "F.Cu" "F.Paste" "F.Mask") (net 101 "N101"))
  (pad "4" smd rect (at -0.525 0.5) (size 0.25 0.85) (layers "F.Cu" "F.Paste" "F.Mask") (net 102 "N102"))
  (pad "4" smd rect (at 0.525 0.5) (size 0.25 0.85) (layers "F.Cu" "F.Paste" "F.Mask") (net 102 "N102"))
  (pad "5" smd rect (at -0.525 1) (size 0.25 0.85) (layers "F.Cu" "F.Paste" "F.Mask") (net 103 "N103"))
  (pad "5" smd rect (at 0.525 1) (size 0.25 0.85) (layers "F.Cu" "F.Paste" "F.Mask") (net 103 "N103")))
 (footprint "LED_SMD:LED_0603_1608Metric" (layer "F.Cu") (at 73.4059 -59.2582)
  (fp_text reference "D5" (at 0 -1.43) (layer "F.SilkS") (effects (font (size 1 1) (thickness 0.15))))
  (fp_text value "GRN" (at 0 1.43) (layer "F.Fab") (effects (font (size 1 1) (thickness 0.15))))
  (fp_line (start -1.485 -0.735) (end -1.485 0.735) (stroke (width 0.12) (type solid)) (layer "F.SilkS"))
  (fp_line (start -1.485 0.735) (end 0.8 0.735) (stroke (width 0.12) (type solid)) (layer "F.SilkS"))
  (fp_line (start 0.8 -0.735) (end -1.485 -0.735) (stroke (width 0.12) (type solid)) (layer "F.SilkS"))
  (pad "1" smd roundrect (at -0.7875 0) (size 0.875 0.95) (layers "F.Cu" "F.Paste" "F.Mask") (roundrect_rratio 0.25) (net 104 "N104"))
  (pad "2" smd roundrect (at 0.7875 0) (size 0.875 0.95) (layers "F.Cu" "F.Paste" "F.Mask") (roundrect_rratio 0.25) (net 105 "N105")))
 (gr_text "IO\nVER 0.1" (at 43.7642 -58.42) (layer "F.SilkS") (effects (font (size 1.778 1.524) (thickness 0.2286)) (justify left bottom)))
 (segment (start -9.5 -11.5066) (end -9.5504 -11.557) (width 0.2794) (layer "B.Cu") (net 3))
 (segment (start -10.5 -3.45) (end -10.5 -11.5922) (width 0.2794) (layer "B.Cu") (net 3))
 (segment (start -11.5 -11.8934) (end -11.4554 -11.938) (width 0.2794) (layer "B.Cu") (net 3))
 (segment (start -8.5 -11.439) (end -8.4582 -11.4808) (width 0.2794) (layer "B.Cu") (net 3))
 (segment (start -11.5 -3.45) (end -11.5 -11.8934) (width 0.2794) (layer "B.Cu") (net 3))
 (segment (start -10.5 -11.5922) (end -10.5156 -11.6078) (width 0.2794) (layer "B.Cu") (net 3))
 (segment (start -8.5 -3.45) (end -8.5 -11.439) (width 0.2794) (layer "B.Cu") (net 3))
 (segment (start -9.5 -3.45) (end -9.5 -11.5066) (width 0.2794) (layer "B.Cu") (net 3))
 (segment (start 10.95 -11.2242) (end 10.922 -11.2522) (width 0.1524) (layer "F.Cu") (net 101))
 (segment (start -10.8966 -7.747) (end -11.5 -7.1436) (width 0.2794) (layer "F.Cu") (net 49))
 (segment (start -9.9822 -7.747) (end -10.8966 -7.747) (width 0.2794) (layer "F.Cu") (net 49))
 (segment (start -9.9822 -7.747) (end -9.0932 -7.747) (width 0.2794) (layer "F.Cu") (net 49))
 (segment (start -8.5 -7.1538) (end -8.5 -3.45) (width 0.2794) (layer "F.Cu") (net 49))
 (segment (start -10.5 -7.7118) (end -10.5 -3.45) (width 0.2794) (layer "F.Cu") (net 49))
 (segment (start -10.4648 -7.747) (end -10.5 -7.7118) (width 0.2794) (layer "F.Cu") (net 49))
 (segment (start -9.9822 -7.747) (end -10.4648 -7.747) (width 0.2794) (layer "F.Cu") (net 49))
 (segment (start -10.0076 -7.8994) (end -10.0076 -12.3698) (width 0.6096) (layer "F.Cu") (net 49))
 (segment (start -9.5 -7.747) (end -9.9822 -7.747) (width 0.2794) (layer "F.Cu") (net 49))
 (segment (start -9.0932 -7.747) (end -8.5 -7.1538) (width 0.2794) (layer "F.Cu") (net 49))
 (segment (start -11.5 -7.1436) (end -11.5 -3.45) (width 0.2794) (layer "F.Cu") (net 49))
 (segment (start -9.5 -3.45) (end -9.5 -7.747) (width 0.2794) (layer "F.Cu") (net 49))
 (segment (start 10.45 -3.5) (end 10.5 -3.45) (width 0.1524) (layer "F.Cu") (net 66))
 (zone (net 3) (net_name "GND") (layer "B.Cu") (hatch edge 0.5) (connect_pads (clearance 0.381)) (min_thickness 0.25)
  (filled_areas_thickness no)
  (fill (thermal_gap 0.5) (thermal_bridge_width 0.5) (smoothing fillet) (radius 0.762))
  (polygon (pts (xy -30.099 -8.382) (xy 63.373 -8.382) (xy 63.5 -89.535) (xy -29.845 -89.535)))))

